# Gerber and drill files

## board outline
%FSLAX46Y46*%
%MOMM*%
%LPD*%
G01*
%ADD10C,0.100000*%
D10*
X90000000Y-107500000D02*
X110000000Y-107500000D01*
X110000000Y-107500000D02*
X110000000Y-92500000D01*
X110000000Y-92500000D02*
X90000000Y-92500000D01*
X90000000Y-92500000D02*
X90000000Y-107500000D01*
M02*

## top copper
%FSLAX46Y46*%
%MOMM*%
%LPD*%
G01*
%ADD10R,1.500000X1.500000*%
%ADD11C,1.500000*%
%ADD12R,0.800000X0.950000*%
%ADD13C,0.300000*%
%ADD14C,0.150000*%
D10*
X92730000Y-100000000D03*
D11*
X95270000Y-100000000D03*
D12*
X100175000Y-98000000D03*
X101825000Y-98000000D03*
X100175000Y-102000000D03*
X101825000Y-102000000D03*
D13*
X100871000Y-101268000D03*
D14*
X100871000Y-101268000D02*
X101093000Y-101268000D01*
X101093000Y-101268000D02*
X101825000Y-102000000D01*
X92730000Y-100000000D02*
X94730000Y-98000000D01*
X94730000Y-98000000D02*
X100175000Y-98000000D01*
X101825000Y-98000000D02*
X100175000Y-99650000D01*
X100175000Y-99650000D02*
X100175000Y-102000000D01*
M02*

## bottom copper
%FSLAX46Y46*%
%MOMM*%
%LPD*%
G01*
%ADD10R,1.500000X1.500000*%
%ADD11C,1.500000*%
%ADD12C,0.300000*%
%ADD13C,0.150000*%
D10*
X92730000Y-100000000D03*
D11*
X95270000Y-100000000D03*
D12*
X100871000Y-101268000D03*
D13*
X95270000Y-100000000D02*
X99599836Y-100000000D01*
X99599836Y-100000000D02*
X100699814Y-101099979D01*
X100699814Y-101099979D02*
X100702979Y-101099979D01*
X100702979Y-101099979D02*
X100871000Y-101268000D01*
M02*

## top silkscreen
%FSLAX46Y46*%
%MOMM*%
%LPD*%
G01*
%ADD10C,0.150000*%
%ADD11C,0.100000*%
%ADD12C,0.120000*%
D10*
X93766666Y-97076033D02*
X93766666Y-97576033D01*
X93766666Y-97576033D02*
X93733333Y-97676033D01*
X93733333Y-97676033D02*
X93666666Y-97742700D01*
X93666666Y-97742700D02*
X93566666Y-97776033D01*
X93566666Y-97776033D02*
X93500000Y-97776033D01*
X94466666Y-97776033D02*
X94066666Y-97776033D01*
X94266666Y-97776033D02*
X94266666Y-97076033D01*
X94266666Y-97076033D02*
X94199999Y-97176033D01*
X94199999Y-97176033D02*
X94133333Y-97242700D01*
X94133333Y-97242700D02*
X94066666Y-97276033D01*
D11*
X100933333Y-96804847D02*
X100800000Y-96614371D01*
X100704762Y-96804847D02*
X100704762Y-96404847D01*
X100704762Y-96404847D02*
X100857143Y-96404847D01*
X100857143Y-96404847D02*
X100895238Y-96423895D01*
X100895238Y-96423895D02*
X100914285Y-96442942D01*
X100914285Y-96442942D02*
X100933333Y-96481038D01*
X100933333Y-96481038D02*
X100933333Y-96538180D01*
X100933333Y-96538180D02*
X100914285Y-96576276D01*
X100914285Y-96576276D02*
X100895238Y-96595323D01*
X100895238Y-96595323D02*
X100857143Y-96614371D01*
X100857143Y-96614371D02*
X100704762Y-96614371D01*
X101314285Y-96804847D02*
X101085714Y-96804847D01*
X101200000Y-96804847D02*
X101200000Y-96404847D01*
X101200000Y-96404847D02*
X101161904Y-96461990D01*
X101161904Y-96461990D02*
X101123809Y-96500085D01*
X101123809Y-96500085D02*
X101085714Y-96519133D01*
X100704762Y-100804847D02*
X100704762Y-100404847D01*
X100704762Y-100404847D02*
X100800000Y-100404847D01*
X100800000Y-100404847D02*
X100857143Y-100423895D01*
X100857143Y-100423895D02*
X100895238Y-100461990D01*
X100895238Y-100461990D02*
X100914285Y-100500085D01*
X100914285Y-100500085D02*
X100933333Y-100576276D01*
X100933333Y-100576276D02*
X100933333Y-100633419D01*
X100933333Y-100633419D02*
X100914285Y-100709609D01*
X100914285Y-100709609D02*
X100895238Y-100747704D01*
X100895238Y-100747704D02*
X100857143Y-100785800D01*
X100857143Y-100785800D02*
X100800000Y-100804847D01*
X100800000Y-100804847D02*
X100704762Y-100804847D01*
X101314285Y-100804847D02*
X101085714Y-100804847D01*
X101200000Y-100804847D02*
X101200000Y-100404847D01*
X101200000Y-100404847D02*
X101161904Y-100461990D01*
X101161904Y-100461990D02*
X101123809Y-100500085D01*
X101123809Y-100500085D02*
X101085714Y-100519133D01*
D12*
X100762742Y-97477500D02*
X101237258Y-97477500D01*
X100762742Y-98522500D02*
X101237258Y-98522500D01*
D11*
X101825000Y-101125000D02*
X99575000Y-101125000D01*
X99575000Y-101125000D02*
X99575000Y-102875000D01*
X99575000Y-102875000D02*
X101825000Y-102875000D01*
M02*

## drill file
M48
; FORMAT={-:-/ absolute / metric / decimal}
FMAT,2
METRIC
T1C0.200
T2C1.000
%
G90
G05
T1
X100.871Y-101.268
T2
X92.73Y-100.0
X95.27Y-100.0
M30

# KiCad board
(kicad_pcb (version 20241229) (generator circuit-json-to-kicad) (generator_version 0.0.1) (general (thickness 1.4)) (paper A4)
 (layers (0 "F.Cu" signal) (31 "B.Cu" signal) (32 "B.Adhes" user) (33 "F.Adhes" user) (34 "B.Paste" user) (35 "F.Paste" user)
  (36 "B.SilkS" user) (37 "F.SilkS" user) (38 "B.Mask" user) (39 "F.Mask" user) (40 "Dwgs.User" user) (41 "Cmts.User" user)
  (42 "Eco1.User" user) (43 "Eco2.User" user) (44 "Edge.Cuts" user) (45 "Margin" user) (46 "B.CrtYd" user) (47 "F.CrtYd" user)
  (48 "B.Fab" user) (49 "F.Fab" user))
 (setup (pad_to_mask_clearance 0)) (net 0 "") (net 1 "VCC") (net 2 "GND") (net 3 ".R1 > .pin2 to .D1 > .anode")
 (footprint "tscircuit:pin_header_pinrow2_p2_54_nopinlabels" (layer F.Cu) (at 94 100 0)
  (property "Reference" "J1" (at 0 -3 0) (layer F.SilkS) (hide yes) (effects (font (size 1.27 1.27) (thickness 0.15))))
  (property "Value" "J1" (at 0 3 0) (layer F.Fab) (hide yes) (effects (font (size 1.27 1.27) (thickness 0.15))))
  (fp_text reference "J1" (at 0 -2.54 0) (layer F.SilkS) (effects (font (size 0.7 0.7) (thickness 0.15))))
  (pad "1" thru_hole rect (at -1.2699999999999996 0 0) (size 1.5 1.5) (drill 1) (layers *.Cu *.Mask) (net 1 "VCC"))
  (pad "2" thru_hole circle (at 1.2699999999999996 0 0) (size 1.5 1.5) (drill 1) (layers *.Cu *.Mask) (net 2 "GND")))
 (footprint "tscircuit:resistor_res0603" (layer F.Cu) (at 101 98 0)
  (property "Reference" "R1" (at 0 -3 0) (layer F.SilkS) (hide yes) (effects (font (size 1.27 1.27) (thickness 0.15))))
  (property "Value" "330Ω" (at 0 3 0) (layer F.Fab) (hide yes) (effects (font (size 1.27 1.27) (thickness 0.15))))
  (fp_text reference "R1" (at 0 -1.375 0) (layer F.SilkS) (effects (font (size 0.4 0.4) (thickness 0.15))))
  (fp_line (start -0.23725799999999997 -0.5225) (end 0.23725799999999997 -0.5225) (stroke (width 0.12) (type default)) (layer F.SilkS))
  (fp_line (start -0.23725799999999997 0.5225) (end 0.23725799999999997 0.5225) (stroke (width 0.12) (type default)) (layer F.SilkS))
  (pad "1" smd rect (at -0.825 0 0) (size 0.8 0.95) (layers F.Cu F.Paste F.Mask) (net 1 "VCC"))
  (pad "2" smd rect (at 0.825 0 0) (size 0.8 0.95) (layers F.Cu F.Paste F.Mask) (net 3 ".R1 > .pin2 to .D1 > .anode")))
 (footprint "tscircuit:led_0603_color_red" (layer F.Cu) (at 101 102 0)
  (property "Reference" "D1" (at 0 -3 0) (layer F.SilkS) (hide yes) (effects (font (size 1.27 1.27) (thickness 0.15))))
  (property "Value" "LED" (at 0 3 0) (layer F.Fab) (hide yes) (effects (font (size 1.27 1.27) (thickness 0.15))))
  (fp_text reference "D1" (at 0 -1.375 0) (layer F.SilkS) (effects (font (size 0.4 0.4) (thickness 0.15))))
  (fp_line (start 0.825 -0.875) (end -1.425 -0.875) (stroke (width 0.1) (type default)) (layer F.SilkS))
  (fp_line (start -1.425 -0.875) (end -1.425 0.875) (stroke (width 0.1) (type default)) (layer F.SilkS))
  (fp_line (start -1.425 0.875) (end 0.825 0.875) (stroke (width 0.1) (type default)) (layer F.SilkS))
  (pad "1" smd rect (at -0.825 0 0) (size 0.8 0.95) (layers F.Cu F.Paste F.Mask) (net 3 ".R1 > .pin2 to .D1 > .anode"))
  (pad "2" smd rect (at 0.825 0 0) (size 0.8 0.95) (layers F.Cu F.Paste F.Mask) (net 2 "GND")))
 (segment (start 95.27 100) (end 99.59983551009537 100) (width 0.15) (layer B.Cu) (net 2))
 (segment (start 99.59983551009537 100) (end 100.6998142288982 101.09997871880282) (width 0.15) (layer B.Cu) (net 2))
 (segment (start 100.6998142288982 101.09997871880282) (end 100.70297871880283 101.09997871880282) (width 0.15) (layer B.Cu) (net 2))
 (segment (start 100.70297871880283 101.09997871880282) (end 100.871 101.268) (width 0.15) (layer B.Cu) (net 2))
 (segment (start 100.871 101.268) (end 101.093 101.268) (width 0.15) (layer F.Cu) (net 2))
 (segment (start 101.093 101.268) (end 101.825 102) (width 0.15) (layer F.Cu) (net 2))
 (segment (start 92.73 100) (end 94.73 98) (width 0.15) (layer F.Cu) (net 1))
 (segment (start 94.73 98) (end 100.175 98) (width 0.15) (layer F.Cu) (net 1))
 (segment (start 101.825 98) (end 100.175 99.65) (width 0.15) (layer F.Cu) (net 3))
 (segment (start 100.175 99.65) (end 100.175 102) (width 0.15) (layer F.Cu) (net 3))
 (gr_line (start 90 107.5) (end 110 107.5) (width 0.1) (layer Edge.Cuts))
 (gr_line (start 110 107.5) (end 110 92.5) (width 0.1) (layer Edge.Cuts))
 (gr_line (start 110 92.5) (end 90 92.5) (width 0.1) (layer Edge.Cuts))
 (gr_line (start 90 92.5) (end 90 107.5) (width 0.1) (layer Edge.Cuts))
 (via (at 100.871 101.268) (size 0.3) (drill 0.2) (layers F.Cu B.Cu) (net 2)))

